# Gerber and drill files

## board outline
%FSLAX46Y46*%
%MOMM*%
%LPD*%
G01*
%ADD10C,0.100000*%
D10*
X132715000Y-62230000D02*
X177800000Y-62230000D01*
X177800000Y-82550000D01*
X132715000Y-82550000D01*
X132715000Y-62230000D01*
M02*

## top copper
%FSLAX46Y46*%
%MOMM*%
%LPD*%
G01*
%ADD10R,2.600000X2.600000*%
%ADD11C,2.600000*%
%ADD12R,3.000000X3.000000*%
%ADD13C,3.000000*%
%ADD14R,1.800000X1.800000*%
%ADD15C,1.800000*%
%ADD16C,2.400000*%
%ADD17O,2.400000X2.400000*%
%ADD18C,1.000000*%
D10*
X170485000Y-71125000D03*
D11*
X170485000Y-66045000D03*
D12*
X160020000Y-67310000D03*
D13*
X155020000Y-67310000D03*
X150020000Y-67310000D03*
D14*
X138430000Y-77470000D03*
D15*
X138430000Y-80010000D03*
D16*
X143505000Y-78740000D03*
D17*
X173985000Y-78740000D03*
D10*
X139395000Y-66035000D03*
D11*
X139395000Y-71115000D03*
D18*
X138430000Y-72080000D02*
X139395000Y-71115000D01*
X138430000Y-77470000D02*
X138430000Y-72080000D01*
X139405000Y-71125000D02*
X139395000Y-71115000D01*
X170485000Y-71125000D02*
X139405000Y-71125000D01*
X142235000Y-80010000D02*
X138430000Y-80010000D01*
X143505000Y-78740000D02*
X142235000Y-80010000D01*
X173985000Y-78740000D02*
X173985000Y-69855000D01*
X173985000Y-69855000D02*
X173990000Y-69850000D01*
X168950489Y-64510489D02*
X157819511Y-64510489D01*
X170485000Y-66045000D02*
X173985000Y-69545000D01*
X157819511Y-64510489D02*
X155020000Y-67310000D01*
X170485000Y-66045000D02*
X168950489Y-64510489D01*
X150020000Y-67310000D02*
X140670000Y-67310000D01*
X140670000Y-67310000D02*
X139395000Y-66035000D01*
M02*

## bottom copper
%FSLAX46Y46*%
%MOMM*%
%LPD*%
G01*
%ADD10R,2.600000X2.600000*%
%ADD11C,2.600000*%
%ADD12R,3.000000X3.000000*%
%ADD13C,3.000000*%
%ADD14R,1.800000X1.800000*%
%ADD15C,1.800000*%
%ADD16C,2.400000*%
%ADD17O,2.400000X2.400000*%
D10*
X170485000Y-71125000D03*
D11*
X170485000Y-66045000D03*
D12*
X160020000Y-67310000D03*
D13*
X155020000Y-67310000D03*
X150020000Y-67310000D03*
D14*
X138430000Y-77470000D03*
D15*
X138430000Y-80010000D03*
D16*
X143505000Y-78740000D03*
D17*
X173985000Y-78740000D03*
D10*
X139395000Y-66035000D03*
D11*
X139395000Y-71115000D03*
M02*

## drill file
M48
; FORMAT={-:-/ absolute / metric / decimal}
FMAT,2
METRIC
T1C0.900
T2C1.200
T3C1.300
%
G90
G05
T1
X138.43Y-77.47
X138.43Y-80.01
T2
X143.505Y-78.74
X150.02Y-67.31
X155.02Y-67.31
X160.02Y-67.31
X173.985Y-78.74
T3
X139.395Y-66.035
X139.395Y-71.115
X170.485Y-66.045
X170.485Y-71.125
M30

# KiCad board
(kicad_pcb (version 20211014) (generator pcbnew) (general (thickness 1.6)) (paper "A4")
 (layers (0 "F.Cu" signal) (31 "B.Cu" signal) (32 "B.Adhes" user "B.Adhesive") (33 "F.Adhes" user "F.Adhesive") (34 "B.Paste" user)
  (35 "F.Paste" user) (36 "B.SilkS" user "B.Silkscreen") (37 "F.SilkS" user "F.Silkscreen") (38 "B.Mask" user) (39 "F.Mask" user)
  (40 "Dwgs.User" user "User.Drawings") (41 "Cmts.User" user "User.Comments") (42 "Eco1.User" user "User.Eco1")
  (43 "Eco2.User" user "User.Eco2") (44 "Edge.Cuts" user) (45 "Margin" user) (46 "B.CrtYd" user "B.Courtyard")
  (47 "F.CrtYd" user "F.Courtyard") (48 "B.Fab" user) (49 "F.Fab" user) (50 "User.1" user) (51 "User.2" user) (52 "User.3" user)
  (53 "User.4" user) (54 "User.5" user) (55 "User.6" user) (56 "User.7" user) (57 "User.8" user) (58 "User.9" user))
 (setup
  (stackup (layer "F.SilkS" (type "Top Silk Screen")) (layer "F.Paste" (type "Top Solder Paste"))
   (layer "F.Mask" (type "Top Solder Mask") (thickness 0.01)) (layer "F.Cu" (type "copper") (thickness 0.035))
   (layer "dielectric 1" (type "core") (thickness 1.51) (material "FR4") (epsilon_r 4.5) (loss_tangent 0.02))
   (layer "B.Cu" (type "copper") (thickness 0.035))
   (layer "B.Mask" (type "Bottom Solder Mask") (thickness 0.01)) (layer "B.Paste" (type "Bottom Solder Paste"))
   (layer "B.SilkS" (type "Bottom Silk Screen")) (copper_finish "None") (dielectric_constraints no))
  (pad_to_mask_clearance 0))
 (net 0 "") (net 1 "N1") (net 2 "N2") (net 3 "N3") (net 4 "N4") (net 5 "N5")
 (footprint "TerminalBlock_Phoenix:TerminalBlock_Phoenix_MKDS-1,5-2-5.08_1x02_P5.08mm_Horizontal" (layer "F.Cu") (at 170.485 71.125 90)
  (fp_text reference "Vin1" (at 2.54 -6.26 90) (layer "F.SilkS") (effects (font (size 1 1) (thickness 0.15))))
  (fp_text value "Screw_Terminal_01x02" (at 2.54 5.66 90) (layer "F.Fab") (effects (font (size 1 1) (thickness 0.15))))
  (pad "1" thru_hole rect (at 0 0 90) (size 2.6 2.6) (drill 1.3) (layers *.Cu *.Mask) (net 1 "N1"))
  (pad "2" thru_hole circle (at 5.08 0 90) (size 2.6 2.6) (drill 1.3) (layers *.Cu *.Mask) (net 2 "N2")))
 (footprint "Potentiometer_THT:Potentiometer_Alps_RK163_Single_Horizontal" (layer "F.Cu") (at 160.02 67.31 -90)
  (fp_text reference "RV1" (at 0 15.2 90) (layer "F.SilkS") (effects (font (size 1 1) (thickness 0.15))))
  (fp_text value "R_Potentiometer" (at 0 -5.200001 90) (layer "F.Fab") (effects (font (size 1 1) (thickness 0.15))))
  (pad "1" thru_hole rect (at 0 0 90) (size 3 3) (drill 1.2) (layers *.Cu *.Mask) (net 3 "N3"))
  (pad "2" thru_hole circle (at 0 5 90) (size 3 3) (drill 1.2) (layers *.Cu *.Mask) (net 2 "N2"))
  (pad "3" thru_hole circle (at 0 10 90) (size 3 3) (drill 1.2) (layers *.Cu *.Mask) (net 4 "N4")))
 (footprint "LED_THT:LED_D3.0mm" (layer "F.Cu") (at 138.43 77.47 -90)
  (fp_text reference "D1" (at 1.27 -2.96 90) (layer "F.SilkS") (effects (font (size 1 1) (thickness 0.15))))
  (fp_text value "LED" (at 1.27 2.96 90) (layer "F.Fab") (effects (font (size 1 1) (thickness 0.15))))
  (pad "1" thru_hole rect (at 0 0 270) (size 1.8 1.8) (drill 0.9) (layers *.Cu *.Mask) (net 1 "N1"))
  (pad "2" thru_hole circle (at 2.54 0 270) (size 1.8 1.8) (drill 0.9) (layers *.Cu *.Mask) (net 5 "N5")))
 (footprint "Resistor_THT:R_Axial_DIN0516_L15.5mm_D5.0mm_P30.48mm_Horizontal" (layer "F.Cu") (at 143.505 78.74)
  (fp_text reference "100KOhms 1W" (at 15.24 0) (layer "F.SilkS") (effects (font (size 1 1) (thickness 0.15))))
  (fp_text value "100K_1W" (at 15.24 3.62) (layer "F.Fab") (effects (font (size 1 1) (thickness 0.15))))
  (pad "1" thru_hole circle (at 0 0) (size 2.4 2.4) (drill 1.2) (layers *.Cu *.Mask) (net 5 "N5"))
  (pad "2" thru_hole oval (at 30.48 0) (size 2.4 2.4) (drill 1.2) (layers *.Cu *.Mask) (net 2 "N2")))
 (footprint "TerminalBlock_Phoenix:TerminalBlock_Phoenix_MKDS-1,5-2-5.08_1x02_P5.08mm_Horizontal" (layer "F.Cu") (at 139.395 66.035 -90)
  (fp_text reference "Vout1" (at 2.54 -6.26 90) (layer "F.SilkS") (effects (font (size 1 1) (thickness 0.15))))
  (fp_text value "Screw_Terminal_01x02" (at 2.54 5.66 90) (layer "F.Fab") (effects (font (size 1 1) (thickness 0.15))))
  (pad "1" thru_hole rect (at 0 0 270) (size 2.6 2.6) (drill 1.3) (layers *.Cu *.Mask) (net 4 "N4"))
  (pad "2" thru_hole circle (at 5.08 0 270) (size 2.6 2.6) (drill 1.3) (layers *.Cu *.Mask) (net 1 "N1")))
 (gr_rect (start 132.715 62.23) (end 177.8 82.55) (layer "Edge.Cuts") (width 0.1) (fill none))
 (segment (start 138.43 72.08) (end 139.395 71.115) (width 1) (layer "F.Cu") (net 1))
 (segment (start 138.43 77.47) (end 138.43 72.08) (width 1) (layer "F.Cu") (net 1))
 (segment (start 139.405 71.125) (end 139.395 71.115) (width 1) (layer "F.Cu") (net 1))
 (segment (start 170.485 71.125) (end 139.405 71.125) (width 1) (layer "F.Cu") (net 1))
 (segment (start 142.235 80.01) (end 138.43 80.01) (width 1) (layer "F.Cu") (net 5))
 (segment (start 143.505 78.74) (end 142.235 80.01) (width 1) (layer "F.Cu") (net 5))
 (segment (start 173.985 78.74) (end 173.985 69.855) (width 1) (layer "F.Cu") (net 2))
 (segment (start 173.985 69.855) (end 173.99 69.85) (width 1) (layer "F.Cu") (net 2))
 (segment (start 168.950489 64.510489) (end 157.819511 64.510489) (width 1) (layer "F.Cu") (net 2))
 (segment (start 170.485 66.045) (end 173.985 69.545) (width 1) (layer "F.Cu") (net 2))
 (segment (start 157.819511 64.510489) (end 155.02 67.31) (width 1) (layer "F.Cu") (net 2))
 (segment (start 170.485 66.045) (end 168.950489 64.510489) (width 1) (layer "F.Cu") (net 2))
 (segment (start 150.02 67.31) (end 140.67 67.31) (width 1) (layer "F.Cu") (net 4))
 (segment (start 140.67 67.31) (end 139.395 66.035) (width 1) (layer "F.Cu") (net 4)))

